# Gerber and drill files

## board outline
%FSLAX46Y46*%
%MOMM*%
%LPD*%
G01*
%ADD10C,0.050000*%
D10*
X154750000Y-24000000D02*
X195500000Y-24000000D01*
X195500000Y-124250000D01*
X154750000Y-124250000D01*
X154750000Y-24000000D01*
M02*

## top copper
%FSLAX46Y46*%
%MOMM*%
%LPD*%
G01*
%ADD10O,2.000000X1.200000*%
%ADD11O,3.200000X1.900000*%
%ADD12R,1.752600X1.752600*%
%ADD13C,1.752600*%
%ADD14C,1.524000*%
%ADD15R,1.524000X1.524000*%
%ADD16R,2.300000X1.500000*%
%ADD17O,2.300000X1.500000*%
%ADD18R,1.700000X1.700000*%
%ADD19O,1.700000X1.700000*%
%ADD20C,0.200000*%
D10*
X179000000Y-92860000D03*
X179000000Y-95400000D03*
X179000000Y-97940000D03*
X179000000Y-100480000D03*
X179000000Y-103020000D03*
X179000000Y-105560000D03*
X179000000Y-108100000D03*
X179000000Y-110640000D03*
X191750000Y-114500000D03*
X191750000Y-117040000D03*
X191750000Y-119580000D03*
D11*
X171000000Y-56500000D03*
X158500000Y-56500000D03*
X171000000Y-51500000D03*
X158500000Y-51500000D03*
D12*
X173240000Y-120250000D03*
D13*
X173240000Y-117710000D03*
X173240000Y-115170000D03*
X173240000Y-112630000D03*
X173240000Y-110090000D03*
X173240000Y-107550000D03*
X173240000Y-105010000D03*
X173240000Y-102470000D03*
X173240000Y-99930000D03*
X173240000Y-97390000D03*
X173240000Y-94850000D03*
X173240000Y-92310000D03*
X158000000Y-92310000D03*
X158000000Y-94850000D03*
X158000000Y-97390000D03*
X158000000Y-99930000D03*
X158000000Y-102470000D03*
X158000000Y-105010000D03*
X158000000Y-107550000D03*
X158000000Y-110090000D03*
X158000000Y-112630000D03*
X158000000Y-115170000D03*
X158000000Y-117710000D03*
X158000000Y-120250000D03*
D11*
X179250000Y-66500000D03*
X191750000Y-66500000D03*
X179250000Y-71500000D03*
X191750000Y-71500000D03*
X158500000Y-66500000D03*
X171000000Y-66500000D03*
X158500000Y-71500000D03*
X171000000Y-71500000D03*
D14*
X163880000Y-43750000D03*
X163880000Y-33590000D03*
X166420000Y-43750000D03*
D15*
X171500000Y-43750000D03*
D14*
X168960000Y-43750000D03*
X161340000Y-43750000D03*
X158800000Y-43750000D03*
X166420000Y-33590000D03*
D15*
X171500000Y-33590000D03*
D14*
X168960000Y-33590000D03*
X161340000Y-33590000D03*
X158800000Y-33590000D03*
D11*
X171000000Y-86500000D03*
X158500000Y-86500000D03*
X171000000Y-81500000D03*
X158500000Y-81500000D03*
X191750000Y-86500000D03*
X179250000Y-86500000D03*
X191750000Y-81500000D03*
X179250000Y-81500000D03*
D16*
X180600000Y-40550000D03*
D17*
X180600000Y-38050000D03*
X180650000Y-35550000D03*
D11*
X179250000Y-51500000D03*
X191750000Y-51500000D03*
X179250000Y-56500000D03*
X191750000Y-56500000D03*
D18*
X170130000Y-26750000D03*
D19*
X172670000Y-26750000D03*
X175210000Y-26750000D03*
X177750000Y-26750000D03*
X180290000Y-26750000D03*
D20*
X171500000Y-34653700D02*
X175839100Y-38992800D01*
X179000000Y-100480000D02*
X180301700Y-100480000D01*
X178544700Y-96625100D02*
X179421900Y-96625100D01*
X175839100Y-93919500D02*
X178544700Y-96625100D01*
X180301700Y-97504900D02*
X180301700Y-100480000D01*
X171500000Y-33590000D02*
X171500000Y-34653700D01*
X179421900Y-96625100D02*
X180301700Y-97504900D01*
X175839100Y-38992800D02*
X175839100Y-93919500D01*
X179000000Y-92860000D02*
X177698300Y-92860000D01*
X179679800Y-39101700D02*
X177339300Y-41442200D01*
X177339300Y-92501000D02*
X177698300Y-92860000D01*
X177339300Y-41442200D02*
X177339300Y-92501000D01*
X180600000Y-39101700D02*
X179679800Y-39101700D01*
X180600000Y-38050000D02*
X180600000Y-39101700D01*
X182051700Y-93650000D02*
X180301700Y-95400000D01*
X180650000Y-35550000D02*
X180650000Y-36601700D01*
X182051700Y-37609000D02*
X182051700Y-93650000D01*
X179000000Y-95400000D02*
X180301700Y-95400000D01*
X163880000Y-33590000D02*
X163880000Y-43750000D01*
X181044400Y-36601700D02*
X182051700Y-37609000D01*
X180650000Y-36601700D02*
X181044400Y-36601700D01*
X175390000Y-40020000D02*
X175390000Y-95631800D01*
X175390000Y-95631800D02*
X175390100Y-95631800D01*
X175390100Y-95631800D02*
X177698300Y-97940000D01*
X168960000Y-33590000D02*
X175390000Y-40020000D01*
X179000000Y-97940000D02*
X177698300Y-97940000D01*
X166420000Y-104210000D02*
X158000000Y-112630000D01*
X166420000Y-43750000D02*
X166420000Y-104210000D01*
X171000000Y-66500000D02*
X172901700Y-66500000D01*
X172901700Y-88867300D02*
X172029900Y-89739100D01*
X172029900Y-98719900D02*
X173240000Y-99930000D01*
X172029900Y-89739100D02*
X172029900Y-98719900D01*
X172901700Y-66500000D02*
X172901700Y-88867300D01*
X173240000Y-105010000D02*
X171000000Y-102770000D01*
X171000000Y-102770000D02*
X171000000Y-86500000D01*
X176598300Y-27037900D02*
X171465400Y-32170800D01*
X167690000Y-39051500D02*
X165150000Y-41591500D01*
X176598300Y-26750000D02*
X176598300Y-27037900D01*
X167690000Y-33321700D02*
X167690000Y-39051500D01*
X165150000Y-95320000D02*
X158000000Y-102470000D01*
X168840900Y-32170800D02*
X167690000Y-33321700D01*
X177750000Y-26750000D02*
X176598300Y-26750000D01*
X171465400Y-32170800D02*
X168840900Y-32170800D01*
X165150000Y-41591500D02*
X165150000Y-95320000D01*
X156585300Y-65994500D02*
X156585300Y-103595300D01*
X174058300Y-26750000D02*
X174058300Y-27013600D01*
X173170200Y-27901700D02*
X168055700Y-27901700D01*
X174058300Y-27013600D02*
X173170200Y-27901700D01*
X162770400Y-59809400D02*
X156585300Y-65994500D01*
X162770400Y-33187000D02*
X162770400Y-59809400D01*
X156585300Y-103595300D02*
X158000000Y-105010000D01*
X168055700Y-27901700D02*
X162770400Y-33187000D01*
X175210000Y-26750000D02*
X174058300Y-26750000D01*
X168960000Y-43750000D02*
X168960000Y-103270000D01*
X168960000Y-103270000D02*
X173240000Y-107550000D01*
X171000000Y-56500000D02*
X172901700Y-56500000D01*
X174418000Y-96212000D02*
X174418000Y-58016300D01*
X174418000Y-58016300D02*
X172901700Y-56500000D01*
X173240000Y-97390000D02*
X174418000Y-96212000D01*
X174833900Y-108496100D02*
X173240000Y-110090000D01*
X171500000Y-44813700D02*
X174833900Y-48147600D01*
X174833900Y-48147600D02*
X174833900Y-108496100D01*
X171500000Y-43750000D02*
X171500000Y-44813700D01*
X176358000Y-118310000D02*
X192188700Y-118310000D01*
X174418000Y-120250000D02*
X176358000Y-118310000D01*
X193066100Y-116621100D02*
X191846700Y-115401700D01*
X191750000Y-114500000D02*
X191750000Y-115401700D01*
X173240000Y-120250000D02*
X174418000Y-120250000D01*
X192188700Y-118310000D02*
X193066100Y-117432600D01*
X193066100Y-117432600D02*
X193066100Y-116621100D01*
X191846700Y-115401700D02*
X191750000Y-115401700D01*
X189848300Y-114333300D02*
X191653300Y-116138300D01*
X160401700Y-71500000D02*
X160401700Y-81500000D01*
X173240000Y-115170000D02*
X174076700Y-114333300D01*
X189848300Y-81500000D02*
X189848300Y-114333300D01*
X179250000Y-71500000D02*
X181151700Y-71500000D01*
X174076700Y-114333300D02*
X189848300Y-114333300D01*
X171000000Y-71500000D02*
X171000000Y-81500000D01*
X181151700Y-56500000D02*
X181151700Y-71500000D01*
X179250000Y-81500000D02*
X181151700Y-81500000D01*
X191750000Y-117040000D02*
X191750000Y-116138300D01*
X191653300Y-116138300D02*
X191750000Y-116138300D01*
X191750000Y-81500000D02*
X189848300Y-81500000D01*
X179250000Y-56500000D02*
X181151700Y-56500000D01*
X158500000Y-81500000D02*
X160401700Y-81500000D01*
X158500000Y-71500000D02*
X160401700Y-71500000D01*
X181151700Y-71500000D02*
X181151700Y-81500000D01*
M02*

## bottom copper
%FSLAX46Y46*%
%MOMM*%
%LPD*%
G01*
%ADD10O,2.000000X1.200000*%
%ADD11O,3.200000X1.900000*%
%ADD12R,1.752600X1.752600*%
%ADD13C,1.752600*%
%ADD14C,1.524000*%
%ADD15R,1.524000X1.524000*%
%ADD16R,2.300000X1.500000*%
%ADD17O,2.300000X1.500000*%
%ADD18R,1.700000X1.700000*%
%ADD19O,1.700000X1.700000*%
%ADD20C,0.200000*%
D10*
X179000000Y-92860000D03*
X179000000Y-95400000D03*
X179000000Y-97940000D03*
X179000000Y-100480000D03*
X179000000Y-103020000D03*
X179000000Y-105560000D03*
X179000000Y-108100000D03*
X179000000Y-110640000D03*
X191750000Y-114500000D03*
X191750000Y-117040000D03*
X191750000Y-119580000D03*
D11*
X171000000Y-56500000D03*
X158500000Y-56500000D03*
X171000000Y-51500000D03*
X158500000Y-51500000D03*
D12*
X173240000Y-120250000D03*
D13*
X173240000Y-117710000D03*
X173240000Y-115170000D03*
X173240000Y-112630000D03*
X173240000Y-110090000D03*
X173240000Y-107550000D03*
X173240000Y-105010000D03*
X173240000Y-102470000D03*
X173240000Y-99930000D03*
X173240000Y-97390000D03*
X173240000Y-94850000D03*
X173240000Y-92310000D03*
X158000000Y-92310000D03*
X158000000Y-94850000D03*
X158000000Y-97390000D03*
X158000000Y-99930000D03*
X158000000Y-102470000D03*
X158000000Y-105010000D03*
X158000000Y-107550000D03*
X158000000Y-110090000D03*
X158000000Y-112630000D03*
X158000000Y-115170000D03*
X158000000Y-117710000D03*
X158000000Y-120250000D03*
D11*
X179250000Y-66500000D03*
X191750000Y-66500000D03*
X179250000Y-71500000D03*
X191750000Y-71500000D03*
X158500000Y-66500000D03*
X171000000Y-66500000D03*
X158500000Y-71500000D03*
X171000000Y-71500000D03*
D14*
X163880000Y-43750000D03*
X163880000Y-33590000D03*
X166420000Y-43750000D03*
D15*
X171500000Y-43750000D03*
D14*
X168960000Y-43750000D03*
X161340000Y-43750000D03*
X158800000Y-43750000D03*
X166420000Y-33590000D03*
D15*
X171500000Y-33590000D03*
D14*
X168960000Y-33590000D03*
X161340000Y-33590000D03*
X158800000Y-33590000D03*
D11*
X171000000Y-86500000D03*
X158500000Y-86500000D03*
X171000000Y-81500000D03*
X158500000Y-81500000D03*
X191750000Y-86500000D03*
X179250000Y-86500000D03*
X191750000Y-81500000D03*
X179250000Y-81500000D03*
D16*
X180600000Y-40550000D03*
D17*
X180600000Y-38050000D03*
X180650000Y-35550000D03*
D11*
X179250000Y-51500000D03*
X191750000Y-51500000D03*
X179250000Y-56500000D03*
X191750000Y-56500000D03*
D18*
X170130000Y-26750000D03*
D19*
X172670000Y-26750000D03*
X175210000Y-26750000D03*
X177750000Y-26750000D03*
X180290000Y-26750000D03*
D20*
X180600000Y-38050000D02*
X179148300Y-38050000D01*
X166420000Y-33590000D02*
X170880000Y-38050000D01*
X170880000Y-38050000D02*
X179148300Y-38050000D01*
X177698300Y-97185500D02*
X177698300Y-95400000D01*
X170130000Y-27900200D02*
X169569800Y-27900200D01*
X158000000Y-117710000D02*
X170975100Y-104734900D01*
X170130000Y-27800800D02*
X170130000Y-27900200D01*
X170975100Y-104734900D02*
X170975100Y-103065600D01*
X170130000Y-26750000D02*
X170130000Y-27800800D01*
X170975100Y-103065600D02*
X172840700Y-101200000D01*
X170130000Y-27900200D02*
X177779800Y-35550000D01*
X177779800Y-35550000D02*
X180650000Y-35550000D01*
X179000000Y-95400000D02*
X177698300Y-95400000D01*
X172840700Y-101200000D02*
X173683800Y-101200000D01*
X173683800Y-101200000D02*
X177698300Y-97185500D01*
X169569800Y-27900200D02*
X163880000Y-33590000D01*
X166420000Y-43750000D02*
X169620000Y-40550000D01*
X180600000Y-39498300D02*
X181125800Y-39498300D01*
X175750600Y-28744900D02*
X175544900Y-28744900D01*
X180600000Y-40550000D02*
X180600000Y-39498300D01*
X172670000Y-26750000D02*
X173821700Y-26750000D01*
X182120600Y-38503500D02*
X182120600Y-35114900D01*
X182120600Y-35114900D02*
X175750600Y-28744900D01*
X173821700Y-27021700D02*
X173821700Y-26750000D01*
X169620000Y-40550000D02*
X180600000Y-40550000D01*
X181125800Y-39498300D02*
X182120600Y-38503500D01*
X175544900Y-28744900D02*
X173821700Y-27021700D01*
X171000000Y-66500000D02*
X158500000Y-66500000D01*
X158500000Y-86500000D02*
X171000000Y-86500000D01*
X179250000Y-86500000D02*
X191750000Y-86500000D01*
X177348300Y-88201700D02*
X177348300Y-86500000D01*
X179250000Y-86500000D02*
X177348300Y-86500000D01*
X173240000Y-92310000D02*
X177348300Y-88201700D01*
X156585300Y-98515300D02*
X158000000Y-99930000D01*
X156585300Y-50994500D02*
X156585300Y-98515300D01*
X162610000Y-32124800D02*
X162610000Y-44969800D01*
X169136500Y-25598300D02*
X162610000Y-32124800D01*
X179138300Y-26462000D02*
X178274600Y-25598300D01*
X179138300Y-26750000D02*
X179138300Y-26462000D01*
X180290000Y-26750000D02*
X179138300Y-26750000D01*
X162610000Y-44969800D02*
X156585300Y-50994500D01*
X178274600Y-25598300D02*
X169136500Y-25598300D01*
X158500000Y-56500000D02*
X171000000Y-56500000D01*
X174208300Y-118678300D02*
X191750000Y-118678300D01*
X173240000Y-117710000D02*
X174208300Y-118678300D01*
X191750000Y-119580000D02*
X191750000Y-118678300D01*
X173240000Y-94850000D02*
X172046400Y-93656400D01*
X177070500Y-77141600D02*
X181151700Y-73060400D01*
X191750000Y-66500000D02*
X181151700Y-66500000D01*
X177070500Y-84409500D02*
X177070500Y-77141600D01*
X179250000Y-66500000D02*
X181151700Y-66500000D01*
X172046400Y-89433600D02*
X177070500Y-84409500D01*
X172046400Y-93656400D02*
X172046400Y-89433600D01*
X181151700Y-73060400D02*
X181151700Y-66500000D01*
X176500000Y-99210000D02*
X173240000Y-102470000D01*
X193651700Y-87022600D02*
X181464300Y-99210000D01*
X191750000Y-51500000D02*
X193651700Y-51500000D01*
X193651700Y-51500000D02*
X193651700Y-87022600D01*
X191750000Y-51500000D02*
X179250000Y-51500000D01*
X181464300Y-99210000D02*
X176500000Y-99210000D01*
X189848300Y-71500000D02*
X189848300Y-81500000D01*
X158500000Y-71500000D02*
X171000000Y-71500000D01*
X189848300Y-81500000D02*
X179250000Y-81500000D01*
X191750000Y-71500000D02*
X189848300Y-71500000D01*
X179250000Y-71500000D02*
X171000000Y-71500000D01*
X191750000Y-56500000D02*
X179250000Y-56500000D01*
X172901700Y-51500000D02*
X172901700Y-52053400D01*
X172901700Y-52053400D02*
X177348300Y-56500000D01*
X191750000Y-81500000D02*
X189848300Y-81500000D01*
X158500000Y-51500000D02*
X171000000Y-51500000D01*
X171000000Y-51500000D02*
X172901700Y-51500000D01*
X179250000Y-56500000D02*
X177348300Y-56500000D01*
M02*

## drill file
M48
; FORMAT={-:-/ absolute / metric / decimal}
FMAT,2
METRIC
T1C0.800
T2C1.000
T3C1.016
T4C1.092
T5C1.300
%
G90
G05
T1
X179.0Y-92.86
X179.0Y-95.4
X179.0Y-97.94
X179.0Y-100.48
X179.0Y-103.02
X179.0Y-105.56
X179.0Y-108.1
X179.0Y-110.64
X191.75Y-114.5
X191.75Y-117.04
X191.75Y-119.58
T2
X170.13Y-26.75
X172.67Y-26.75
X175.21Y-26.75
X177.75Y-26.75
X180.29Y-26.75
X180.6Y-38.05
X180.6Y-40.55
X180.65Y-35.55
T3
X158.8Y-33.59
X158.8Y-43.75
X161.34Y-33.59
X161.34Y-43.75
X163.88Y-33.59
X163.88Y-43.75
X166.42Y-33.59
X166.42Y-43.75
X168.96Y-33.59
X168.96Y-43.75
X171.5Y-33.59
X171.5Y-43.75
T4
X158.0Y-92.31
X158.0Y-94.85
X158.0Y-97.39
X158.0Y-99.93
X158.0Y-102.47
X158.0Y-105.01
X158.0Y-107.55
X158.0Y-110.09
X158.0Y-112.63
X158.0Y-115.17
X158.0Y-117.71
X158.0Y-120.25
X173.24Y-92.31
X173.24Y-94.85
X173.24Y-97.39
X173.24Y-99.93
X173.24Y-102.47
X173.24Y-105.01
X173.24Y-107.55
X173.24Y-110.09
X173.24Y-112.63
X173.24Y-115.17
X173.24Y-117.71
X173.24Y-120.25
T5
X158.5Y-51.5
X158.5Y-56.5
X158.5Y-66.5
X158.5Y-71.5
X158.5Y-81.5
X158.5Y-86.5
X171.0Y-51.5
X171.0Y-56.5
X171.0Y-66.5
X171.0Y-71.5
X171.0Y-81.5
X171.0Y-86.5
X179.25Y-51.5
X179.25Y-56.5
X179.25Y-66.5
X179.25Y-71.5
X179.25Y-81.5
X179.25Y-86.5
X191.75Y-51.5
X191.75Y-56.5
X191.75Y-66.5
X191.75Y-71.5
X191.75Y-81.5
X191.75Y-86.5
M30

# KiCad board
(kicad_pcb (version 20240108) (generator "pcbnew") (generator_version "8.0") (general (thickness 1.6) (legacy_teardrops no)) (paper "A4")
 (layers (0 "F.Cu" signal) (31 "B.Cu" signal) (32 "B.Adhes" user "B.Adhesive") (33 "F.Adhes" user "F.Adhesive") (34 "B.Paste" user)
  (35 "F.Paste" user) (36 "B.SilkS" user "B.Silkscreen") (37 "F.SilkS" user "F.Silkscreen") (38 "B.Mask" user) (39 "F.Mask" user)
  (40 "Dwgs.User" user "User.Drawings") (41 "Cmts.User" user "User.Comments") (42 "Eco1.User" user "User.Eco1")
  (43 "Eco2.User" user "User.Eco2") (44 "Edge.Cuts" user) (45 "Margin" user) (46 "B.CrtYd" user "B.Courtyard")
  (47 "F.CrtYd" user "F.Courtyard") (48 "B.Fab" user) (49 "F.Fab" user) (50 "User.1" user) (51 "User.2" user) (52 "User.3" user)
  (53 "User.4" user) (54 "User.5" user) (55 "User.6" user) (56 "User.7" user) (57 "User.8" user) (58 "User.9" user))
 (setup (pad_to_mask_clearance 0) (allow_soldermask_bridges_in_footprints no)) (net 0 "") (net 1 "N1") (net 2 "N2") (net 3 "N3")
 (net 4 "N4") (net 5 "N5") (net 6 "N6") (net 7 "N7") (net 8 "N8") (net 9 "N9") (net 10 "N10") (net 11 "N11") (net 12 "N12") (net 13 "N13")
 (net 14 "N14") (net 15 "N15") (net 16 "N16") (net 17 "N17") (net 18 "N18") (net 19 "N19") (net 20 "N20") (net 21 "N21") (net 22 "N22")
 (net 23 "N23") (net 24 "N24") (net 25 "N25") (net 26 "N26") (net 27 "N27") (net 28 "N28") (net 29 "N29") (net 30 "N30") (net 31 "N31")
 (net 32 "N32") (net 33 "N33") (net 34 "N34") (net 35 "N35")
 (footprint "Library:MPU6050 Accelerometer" (layer "F.Cu") (at 185.5 104)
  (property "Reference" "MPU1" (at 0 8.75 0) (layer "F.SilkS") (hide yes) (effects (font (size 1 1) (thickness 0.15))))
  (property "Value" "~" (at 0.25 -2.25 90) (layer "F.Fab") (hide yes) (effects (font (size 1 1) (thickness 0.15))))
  (pad "1" thru_hole oval (at -6.5 -11.14 270) (size 1.2 2) (drill 0.8) (layers "*.Cu" "*.Mask") (remove_unused_layers no) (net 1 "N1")
   (thermal_bridge_angle 45))
  (pad "2" thru_hole oval (at -6.5 -8.6 270) (size 1.2 2) (drill 0.8) (layers "*.Cu" "*.Mask") (remove_unused_layers no) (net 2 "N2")
   (thermal_bridge_angle 45))
  (pad "3" thru_hole oval (at -6.5 -6.06 270) (size 1.2 2) (drill 0.8) (layers "*.Cu" "*.Mask") (remove_unused_layers no) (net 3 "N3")
   (thermal_bridge_angle 45))
  (pad "4" thru_hole oval (at -6.5 -3.52 270) (size 1.2 2) (drill 0.8) (layers "*.Cu" "*.Mask") (remove_unused_layers no) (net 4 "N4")
   (thermal_bridge_angle 45))
  (pad "5" thru_hole oval (at -6.5 -0.98 270) (size 1.2 2) (drill 0.8) (layers "*.Cu" "*.Mask") (remove_unused_layers no) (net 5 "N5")
   (thermal_bridge_angle 45))
  (pad "6" thru_hole oval (at -6.5 1.56 270) (size 1.2 2) (drill 0.8) (layers "*.Cu" "*.Mask") (remove_unused_layers no) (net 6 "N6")
   (thermal_bridge_angle 45))
  (pad "7" thru_hole oval (at -6.5 4.1 270) (size 1.2 2) (drill 0.8) (layers "*.Cu" "*.Mask") (remove_unused_layers no) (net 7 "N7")
   (thermal_bridge_angle 45))
  (pad "8" thru_hole oval (at -6.5 6.64 270) (size 1.2 2) (drill 0.8) (layers "*.Cu" "*.Mask") (remove_unused_layers no) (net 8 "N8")
   (thermal_bridge_angle 45)))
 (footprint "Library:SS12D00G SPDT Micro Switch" (layer "F.Cu") (at 191.75 117.04 -90)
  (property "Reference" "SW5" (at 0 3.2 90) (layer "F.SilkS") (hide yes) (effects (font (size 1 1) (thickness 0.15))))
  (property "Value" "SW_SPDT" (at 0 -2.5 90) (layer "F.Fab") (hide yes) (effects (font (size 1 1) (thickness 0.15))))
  (pad "1" thru_hole oval (at -2.54 0 270) (size 1.2 2) (drill 0.8) (layers "*.Cu" "*.Mask") (remove_unused_layers no) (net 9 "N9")
   (thermal_bridge_angle 45))
  (pad "2" thru_hole oval (at 0 0 270) (size 1.2 2) (drill 0.8) (layers "*.Cu" "*.Mask") (remove_unused_layers no) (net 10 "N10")
   (thermal_bridge_angle 45))
  (pad "3" thru_hole oval (at 2.54 0 270) (size 1.2 2) (drill 0.8) (layers "*.Cu" "*.Mask") (remove_unused_layers no) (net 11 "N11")
   (thermal_bridge_angle 45)))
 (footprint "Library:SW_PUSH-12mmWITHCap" (layer "F.Cu") (at 171 56.5 180)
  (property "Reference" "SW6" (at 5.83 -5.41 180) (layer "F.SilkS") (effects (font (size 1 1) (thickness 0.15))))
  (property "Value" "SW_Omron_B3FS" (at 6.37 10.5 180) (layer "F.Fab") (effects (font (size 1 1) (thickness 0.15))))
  (pad "1" thru_hole oval (at 0 0 180) (size 3.2 1.9) (drill 1.3) (layers "*.Cu" "*.Mask") (remove_unused_layers no) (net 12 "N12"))
  (pad "1" thru_hole oval (at 12.5 0 180) (size 3.2 1.9) (drill 1.3) (layers "*.Cu" "*.Mask") (remove_unused_layers no) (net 12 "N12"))
  (pad "2" thru_hole oval (at 0 5 180) (size 3.2 1.9) (drill 1.3) (layers "*.Cu" "*.Mask") (remove_unused_layers no) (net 10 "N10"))
  (pad "2" thru_hole oval (at 12.5 5 180) (size 3.2 1.9) (drill 1.3) (layers "*.Cu" "*.Mask") (remove_unused_layers no) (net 10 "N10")))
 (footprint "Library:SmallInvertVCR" (layer "F.Cu") (at 182.25 117.5)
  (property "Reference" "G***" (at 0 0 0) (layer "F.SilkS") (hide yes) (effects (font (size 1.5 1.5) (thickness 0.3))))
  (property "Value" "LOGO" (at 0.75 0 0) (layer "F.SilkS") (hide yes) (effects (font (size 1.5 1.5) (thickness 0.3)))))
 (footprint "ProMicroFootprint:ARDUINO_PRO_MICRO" (layer "F.Cu") (at 165.62 106.28 90)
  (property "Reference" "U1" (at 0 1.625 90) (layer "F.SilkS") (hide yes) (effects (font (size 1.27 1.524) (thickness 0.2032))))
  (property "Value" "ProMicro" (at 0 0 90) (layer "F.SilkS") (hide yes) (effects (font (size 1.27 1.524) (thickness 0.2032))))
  (pad "1" thru_hole rect (at -13.97 7.62 90) (size 1.7526 1.7526) (drill 1.0922) (layers "*.Cu" "*.SilkS" "*.Mask")
   (remove_unused_layers no) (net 9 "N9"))
  (pad "2" thru_hole circle (at -11.43 7.62 90) (size 1.7526 1.7526) (drill 1.0922) (layers "*.Cu" "*.SilkS" "*.Mask")
   (remove_unused_layers no) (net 11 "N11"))
  (pad "3" thru_hole circle (at -8.89 7.62 90) (size 1.7526 1.7526) (drill 1.0922) (layers "*.Cu" "*.SilkS" "*.Mask")
   (remove_unused_layers no) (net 10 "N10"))
  (pad "4" thru_hole circle (at -6.35 7.62 90) (size 1.7526 1.7526) (drill 1.0922) (layers "*.Cu" "*.SilkS" "*.Mask")
   (remove_unused_layers no) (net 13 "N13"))
  (pad "5" thru_hole circle (at -3.81 7.62 90) (size 1.7526 1.7526) (drill 1.0922) (layers "*.Cu" "*.SilkS" "*.Mask")
   (remove_unused_layers no) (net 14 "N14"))
  (pad "6" thru_hole circle (at -1.27 7.62 90) (size 1.7526 1.7526) (drill 1.0922) (layers "*.Cu" "*.SilkS" "*.Mask")
   (remove_unused_layers no) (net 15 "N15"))
  (pad "7" thru_hole circle (at 1.27 7.62 90) (size 1.7526 1.7526) (drill 1.0922) (layers "*.Cu" "*.SilkS" "*.Mask")
   (remove_unused_layers no) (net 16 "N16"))
  (pad "8" thru_hole circle (at 3.81 7.62 90) (size 1.7526 1.7526) (drill 1.0922) (layers "*.Cu" "*.SilkS" "*.Mask")
   (remove_unused_layers no) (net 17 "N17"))
  (pad "9" thru_hole circle (at 6.35 7.62 90) (size 1.7526 1.7526) (drill 1.0922) (layers "*.Cu" "*.SilkS" "*.Mask")
   (remove_unused_layers no) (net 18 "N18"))
  (pad "10" thru_hole circle (at 8.89 7.62 90) (size 1.7526 1.7526) (drill 1.0922) (layers "*.Cu" "*.SilkS" "*.Mask")
   (remove_unused_layers no) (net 12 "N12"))
  (pad "11" thru_hole circle (at 11.43 7.62 90) (size 1.7526 1.7526) (drill 1.0922) (layers "*.Cu" "*.SilkS" "*.Mask")
   (remove_unused_layers no) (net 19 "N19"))
  (pad "12" thru_hole circle (at 13.97 7.62 90) (size 1.7526 1.7526) (drill 1.0922) (layers "*.Cu" "*.SilkS" "*.Mask")
   (remove_unused_layers no) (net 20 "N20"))
  (pad "13" thru_hole circle (at 13.97 -7.62 90) (size 1.7526 1.7526) (drill 1.0922) (layers "*.Cu" "*.SilkS" "*.Mask")
   (remove_unused_layers no) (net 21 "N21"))
  (pad "14" thru_hole circle (at 11.43 -7.62 90) (size 1.7526 1.7526) (drill 1.0922) (layers "*.Cu" "*.SilkS" "*.Mask")
   (remove_unused_layers no) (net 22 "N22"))
  (pad "15" thru_hole circle (at 8.89 -7.62 90) (size 1.7526 1.7526) (drill 1.0922) (layers "*.Cu" "*.SilkS" "*.Mask")
   (remove_unused_layers no) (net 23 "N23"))
  (pad "16" thru_hole circle (at 6.35 -7.62 90) (size 1.7526 1.7526) (drill 1.0922) (layers "*.Cu" "*.SilkS" "*.Mask")
   (remove_unused_layers no) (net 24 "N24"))
  (pad "17" thru_hole circle (at 3.81 -7.62 90) (size 1.7526 1.7526) (drill 1.0922) (layers "*.Cu" "*.SilkS" "*.Mask")
   (remove_unused_layers no) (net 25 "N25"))
  (pad "18" thru_hole circle (at 1.27 -7.62 90) (size 1.7526 1.7526) (drill 1.0922) (layers "*.Cu" "*.SilkS" "*.Mask")
   (remove_unused_layers no) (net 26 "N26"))
  (pad "19" thru_hole circle (at -1.27 -7.62 90) (size 1.7526 1.7526) (drill 1.0922) (layers "*.Cu" "*.SilkS" "*.Mask")
   (remove_unused_layers no) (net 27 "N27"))
  (pad "20" thru_hole circle (at -3.81 -7.62 90) (size 1.7526 1.7526) (drill 1.0922) (layers "*.Cu" "*.SilkS" "*.Mask")
   (remove_unused_layers no) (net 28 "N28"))
  (pad "21" thru_hole circle (at -6.35 -7.62 90) (size 1.7526 1.7526) (drill 1.0922) (layers "*.Cu" "*.SilkS" "*.Mask")
   (remove_unused_layers no) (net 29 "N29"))
  (pad "22" thru_hole circle (at -8.89 -7.62 90) (size 1.7526 1.7526) (drill 1.0922) (layers "*.Cu" "*.SilkS" "*.Mask")
   (remove_unused_layers no) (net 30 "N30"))
  (pad "23" thru_hole circle (at -11.43 -7.62 90) (size 1.7526 1.7526) (drill 1.0922) (layers "*.Cu" "*.SilkS" "*.Mask")
   (remove_unused_layers no) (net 2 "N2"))
  (pad "24" thru_hole circle (at -13.97 -7.62 90) (size 1.7526 1.7526) (drill 1.0922) (layers "*.Cu" "*.SilkS" "*.Mask")
   (remove_unused_layers no) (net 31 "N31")))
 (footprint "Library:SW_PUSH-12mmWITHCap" (layer "F.Cu") (at 179.25 66.5)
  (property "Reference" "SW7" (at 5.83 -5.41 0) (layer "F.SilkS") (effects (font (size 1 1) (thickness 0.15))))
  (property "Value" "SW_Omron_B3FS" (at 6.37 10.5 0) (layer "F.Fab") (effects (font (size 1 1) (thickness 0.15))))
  (pad "1" thru_hole oval (at 0 0) (size 3.2 1.9) (drill 1.3) (layers "*.Cu" "*.Mask") (remove_unused_layers no) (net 19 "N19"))
  (pad "1" thru_hole oval (at 12.5 0) (size 3.2 1.9) (drill 1.3) (layers "*.Cu" "*.Mask") (remove_unused_layers no) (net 19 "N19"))
  (pad "2" thru_hole oval (at 0 5) (size 3.2 1.9) (drill 1.3) (layers "*.Cu" "*.Mask") (remove_unused_layers no) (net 10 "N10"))
  (pad "2" thru_hole oval (at 12.5 5) (size 3.2 1.9) (drill 1.3) (layers "*.Cu" "*.Mask") (remove_unused_layers no) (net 10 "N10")))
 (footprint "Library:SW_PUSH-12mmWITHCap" (layer "F.Cu") (at 158.5 66.5)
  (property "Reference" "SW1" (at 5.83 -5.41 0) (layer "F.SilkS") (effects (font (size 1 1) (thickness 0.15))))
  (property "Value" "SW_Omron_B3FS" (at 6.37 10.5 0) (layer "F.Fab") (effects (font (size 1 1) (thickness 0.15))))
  (pad "1" thru_hole oval (at 0 0) (size 3.2 1.9) (drill 1.3) (layers "*.Cu" "*.Mask") (remove_unused_layers no) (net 18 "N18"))
  (pad "1" thru_hole oval (at 12.5 0) (size 3.2 1.9) (drill 1.3) (layers "*.Cu" "*.Mask") (remove_unused_layers no) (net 18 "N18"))
  (pad "2" thru_hole oval (at 0 5) (size 3.2 1.9) (drill 1.3) (layers "*.Cu" "*.Mask") (remove_unused_layers no) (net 10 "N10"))
  (pad "2" thru_hole oval (at 12.5 5) (size 3.2 1.9) (drill 1.3) (layers "*.Cu" "*.Mask") (remove_unused_layers no) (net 10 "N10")))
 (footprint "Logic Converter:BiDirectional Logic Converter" (layer "F.Cu") (at 165.15 38.67 -90)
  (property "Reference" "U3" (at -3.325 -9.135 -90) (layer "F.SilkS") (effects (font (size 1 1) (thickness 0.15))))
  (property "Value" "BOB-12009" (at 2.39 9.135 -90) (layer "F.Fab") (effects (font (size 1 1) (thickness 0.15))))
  (pad "GND_1" thru_hole circle (at 5.08 1.27 270) (size 1.524 1.524) (drill 1.016) (layers "*.Cu" "*.Mask") (remove_unused_layers no)
   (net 2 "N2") (solder_mask_margin 0.102))
  (pad "GND_2" thru_hole circle (at -5.08 1.27 270) (size 1.524 1.524) (drill 1.016) (layers "*.Cu" "*.Mask") (remove_unused_layers no)
   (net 2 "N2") (solder_mask_margin 0.102))
  (pad "HV" thru_hole circle (at 5.08 -1.27 270) (size 1.524 1.524) (drill 1.016) (layers "*.Cu" "*.Mask") (remove_unused_layers no)
   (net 29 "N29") (solder_mask_margin 0.102))
  (pad "HV1" thru_hole rect (at 5.08 -6.35 270) (size 1.524 1.524) (drill 1.016) (layers "*.Cu" "*.Mask") (remove_unused_layers no)
   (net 14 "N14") (solder_mask_margin 0.102))
  (pad "HV2" thru_hole circle (at 5.08 -3.81 270) (size 1.524 1.524) (drill 1.016) (layers "*.Cu" "*.Mask") (remove_unused_layers no)
   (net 15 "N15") (solder_mask_margin 0.102))
  (pad "HV3" thru_hole circle (at 5.08 3.81 270) (size 1.524 1.524) (drill 1.016) (layers "*.Cu" "*.Mask") (remove_unused_layers no)
   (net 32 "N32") (solder_mask_margin 0.102))
  (pad "HV4" thru_hole circle (at 5.08 6.35 270) (size 1.524 1.524) (drill 1.016) (layers "*.Cu" "*.Mask") (remove_unused_layers no)
   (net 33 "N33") (solder_mask_margin 0.102))
  (pad "LV" thru_hole circle (at -5.08 -1.27 270) (size 1.524 1.524) (drill 1.016) (layers "*.Cu" "*.Mask") (remove_unused_layers no)
   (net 1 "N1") (solder_mask_margin 0.102))
  (pad "LV1" thru_hole rect (at -5.08 -6.35 270) (size 1.524 1.524) (drill 1.016) (layers "*.Cu" "*.Mask") (remove_unused_layers no)
   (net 4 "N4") (solder_mask_margin 0.102))
  (pad "LV2" thru_hole circle (at -5.08 -3.81 270) (size 1.524 1.524) (drill 1.016) (layers "*.Cu" "*.Mask") (remove_unused_layers no)
   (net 3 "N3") (solder_mask_margin 0.102))
  (pad "LV3" thru_hole circle (at -5.08 3.81 270) (size 1.524 1.524) (drill 1.016) (layers "*.Cu" "*.Mask") (remove_unused_layers no)
   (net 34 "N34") (solder_mask_margin 0.102))
  (pad "LV4" thru_hole circle (at -5.08 6.35 270) (size 1.524 1.524) (drill 1.016) (layers "*.Cu" "*.Mask") (remove_unused_layers no)
   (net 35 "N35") (solder_mask_margin 0.102)))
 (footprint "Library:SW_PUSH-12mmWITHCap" (layer "F.Cu") (at 171 86.5 180)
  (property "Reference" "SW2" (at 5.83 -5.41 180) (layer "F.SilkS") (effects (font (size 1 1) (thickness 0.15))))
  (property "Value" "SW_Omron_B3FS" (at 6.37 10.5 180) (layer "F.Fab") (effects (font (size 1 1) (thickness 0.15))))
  (pad "1" thru_hole oval (at 0 0 180) (size 3.2 1.9) (drill 1.3) (layers "*.Cu" "*.Mask") (remove_unused_layers no) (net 16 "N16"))
  (pad "1" thru_hole oval (at 12.5 0 180) (size 3.2 1.9) (drill 1.3) (layers "*.Cu" "*.Mask") (remove_unused_layers no) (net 16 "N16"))
  (pad "2" thru_hole oval (at 0 5 180) (size 3.2 1.9) (drill 1.3) (layers "*.Cu" "*.Mask") (remove_unused_layers no) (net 10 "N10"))
  (pad "2" thru_hole oval (at 12.5 5 180) (size 3.2 1.9) (drill 1.3) (layers "*.Cu" "*.Mask") (remove_unused_layers no) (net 10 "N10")))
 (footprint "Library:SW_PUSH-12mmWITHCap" (layer "F.Cu") (at 191.75 86.5 180)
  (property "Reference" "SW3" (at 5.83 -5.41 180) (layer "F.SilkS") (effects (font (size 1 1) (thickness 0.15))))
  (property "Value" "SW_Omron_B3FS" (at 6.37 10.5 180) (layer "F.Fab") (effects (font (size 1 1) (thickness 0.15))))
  (pad "1" thru_hole oval (at 0 0 180) (size 3.2 1.9) (drill 1.3) (layers "*.Cu" "*.Mask") (remove_unused_layers no) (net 20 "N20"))
  (pad "1" thru_hole oval (at 12.5 0 180) (size 3.2 1.9) (drill 1.3) (layers "*.Cu" "*.Mask") (remove_unused_layers no) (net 20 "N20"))
  (pad "2" thru_hole oval (at 0 5 180) (size 3.2 1.9) (drill 1.3) (layers "*.Cu" "*.Mask") (remove_unused_layers no) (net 10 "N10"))
  (pad "2" thru_hole oval (at 12.5 5 180) (size 3.2 1.9) (drill 1.3) (layers "*.Cu" "*.Mask") (remove_unused_layers no) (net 10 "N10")))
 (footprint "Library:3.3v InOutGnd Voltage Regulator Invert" (layer "F.Cu") (at 179.1 38 -90)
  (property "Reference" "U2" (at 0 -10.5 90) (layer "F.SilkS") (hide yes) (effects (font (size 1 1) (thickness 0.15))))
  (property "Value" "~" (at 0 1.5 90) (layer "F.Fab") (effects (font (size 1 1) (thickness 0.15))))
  (pad "1" thru_hole rect (at 2.55 -1.5 270) (size 1.5 2.3) (drill 1) (layers "*.Cu" "*.Mask") (remove_unused_layers no) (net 29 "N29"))
  (pad "2" thru_hole oval (at 0.05 -1.5 270) (size 1.5 2.3) (drill 1) (layers "*.Cu" "*.Mask") (remove_unused_layers no) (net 1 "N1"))
  (pad "3" thru_hole oval (at -2.45 -1.55 270) (size 1.5 2.3) (drill 1) (layers "*.Cu" "*.Mask") (remove_unused_layers no) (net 2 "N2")))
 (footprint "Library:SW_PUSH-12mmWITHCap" (layer "F.Cu") (at 179.25 51.5)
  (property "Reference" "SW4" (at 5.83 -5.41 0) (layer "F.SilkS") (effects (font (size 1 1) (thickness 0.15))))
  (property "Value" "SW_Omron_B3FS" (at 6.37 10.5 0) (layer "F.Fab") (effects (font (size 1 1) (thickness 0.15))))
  (pad "1" thru_hole oval (at 0 0) (size 3.2 1.9) (drill 1.3) (layers "*.Cu" "*.Mask") (remove_unused_layers no) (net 17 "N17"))
  (pad "1" thru_hole oval (at 12.5 0) (size 3.2 1.9) (drill 1.3) (layers "*.Cu" "*.Mask") (remove_unused_layers no) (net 17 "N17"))
  (pad "2" thru_hole oval (at 0 5) (size 3.2 1.9) (drill 1.3) (layers "*.Cu" "*.Mask") (remove_unused_layers no) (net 10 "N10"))
  (pad "2" thru_hole oval (at 12.5 5) (size 3.2 1.9) (drill 1.3) (layers "*.Cu" "*.Mask") (remove_unused_layers no) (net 10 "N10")))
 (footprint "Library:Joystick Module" (layer "B.Cu") (at 170.13 26.75 -90)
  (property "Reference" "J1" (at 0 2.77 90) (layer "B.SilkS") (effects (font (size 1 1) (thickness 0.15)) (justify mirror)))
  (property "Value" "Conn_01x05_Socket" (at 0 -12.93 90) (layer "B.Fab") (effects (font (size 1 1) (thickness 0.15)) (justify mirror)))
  (pad "1" thru_hole rect (at 0 0 270) (size 1.7 1.7) (drill 1) (layers "*.Cu" "*.Mask") (remove_unused_layers no) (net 2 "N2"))
  (pad "2" thru_hole oval (at 0 -2.54 270) (size 1.7 1.7) (drill 1) (layers "*.Cu" "*.Mask") (remove_unused_layers no) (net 29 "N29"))
  (pad "3" thru_hole oval (at 0 -5.08 270) (size 1.7 1.7) (drill 1) (layers "*.Cu" "*.Mask") (remove_unused_layers no) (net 26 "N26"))
  (pad "4" thru_hole oval (at 0 -7.62 270) (size 1.7 1.7) (drill 1) (layers "*.Cu" "*.Mask") (remove_unused_layers no) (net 25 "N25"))
  (pad "5" thru_hole oval (at 0 -10.16 270) (size 1.7 1.7) (drill 1) (layers "*.Cu" "*.Mask") (remove_unused_layers no) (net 24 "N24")))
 (gr_rect (start 154.75 24) (end 195.5 124.25) (stroke (width 0.05) (type default)) (fill none) (layer "Edge.Cuts"))
 (segment (start 171.5 34.6537) (end 175.8391 38.9928) (width 0.2) (layer "F.Cu") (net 4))
 (segment (start 179 100.48) (end 180.3017 100.48) (width 0.2) (layer "F.Cu") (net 4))
 (segment (start 178.5447 96.6251) (end 179.4219 96.6251) (width 0.2) (layer "F.Cu") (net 4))
 (segment (start 175.8391 93.9195) (end 178.5447 96.6251) (width 0.2) (layer "F.Cu") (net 4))
 (segment (start 180.3017 97.5049) (end 180.3017 100.48) (width 0.2) (layer "F.Cu") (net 4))
 (segment (start 171.5 33.59) (end 171.5 34.6537) (width 0.2) (layer "F.Cu") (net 4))
 (segment (start 179.4219 96.6251) (end 180.3017 97.5049) (width 0.2) (layer "F.Cu") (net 4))
 (segment (start 175.8391 38.9928) (end 175.8391 93.9195) (width 0.2) (layer "F.Cu") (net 4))
 (segment (start 179 92.86) (end 177.6983 92.86) (width 0.2) (layer "F.Cu") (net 1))
 (segment (start 179.6798 39.1017) (end 177.3393 41.4422) (width 0.2) (layer "F.Cu") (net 1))
 (segment (start 177.3393 92.501) (end 177.6983 92.86) (width 0.2) (layer "F.Cu") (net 1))
 (segment (start 177.3393 41.4422) (end 177.3393 92.501) (width 0.2) (layer "F.Cu") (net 1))
 (segment (start 180.6 39.1017) (end 179.6798 39.1017) (width 0.2) (layer "F.Cu") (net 1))
 (segment (start 180.6 38.05) (end 180.6 39.1017) (width 0.2) (layer "F.Cu") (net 1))
 (segment (start 180.6 38.05) (end 179.1483 38.05) (width 0.2) (layer "B.Cu") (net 1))
 (segment (start 166.42 33.59) (end 170.88 38.05) (width 0.2) (layer "B.Cu") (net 1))
 (segment (start 170.88 38.05) (end 179.1483 38.05) (width 0.2) (layer "B.Cu") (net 1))
 (segment (start 182.0517 93.65) (end 180.3017 95.4) (width 0.2) (layer "F.Cu") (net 2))
 (segment (start 180.65 35.55) (end 180.65 36.6017) (width 0.2) (layer "F.Cu") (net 2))
 (segment (start 182.0517 37.609) (end 182.0517 93.65) (width 0.2) (layer "F.Cu") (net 2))
 (segment (start 179 95.4) (end 180.3017 95.4) (width 0.2) (layer "F.Cu") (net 2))
 (segment (start 163.88 33.59) (end 163.88 43.75) (width 0.2) (layer "F.Cu") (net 2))
 (segment (start 181.0444 36.6017) (end 182.0517 37.609) (width 0.2) (layer "F.Cu") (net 2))
 (segment (start 180.65 36.6017) (end 181.0444 36.6017) (width 0.2) (layer "F.Cu") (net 2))
 (segment (start 177.6983 97.1855) (end 177.6983 95.4) (width 0.2) (layer "B.Cu") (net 2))
 (segment (start 170.13 27.9002) (end 169.5698 27.9002) (width 0.2) (layer "B.Cu") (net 2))
 (segment (start 158 117.71) (end 170.9751 104.7349) (width 0.2) (layer "B.Cu") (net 2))
 (segment (start 170.13 27.8008) (end 170.13 27.9002) (width 0.2) (layer "B.Cu") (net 2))
 (segment (start 170.9751 104.7349) (end 170.9751 103.0656) (width 0.2) (layer "B.Cu") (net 2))
 (segment (start 170.13 26.75) (end 170.13 27.8008) (width 0.2) (layer "B.Cu") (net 2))
 (segment (start 170.9751 103.0656) (end 172.8407 101.2) (width 0.2) (layer "B.Cu") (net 2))
 (segment (start 170.13 27.9002) (end 177.7798 35.55) (width 0.2) (layer "B.Cu") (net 2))
 (segment (start 177.7798 35.55) (end 180.65 35.55) (width 0.2) (layer "B.Cu") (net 2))
 (segment (start 179 95.4) (end 177.6983 95.4) (width 0.2) (layer "B.Cu") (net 2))
 (segment (start 172.8407 101.2) (end 173.6838 101.2) (width 0.2) (layer "B.Cu") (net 2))
 (segment (start 173.6838 101.2) (end 177.6983 97.1855) (width 0.2) (layer "B.Cu") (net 2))
 (segment (start 169.5698 27.9002) (end 163.88 33.59) (width 0.2) (layer "B.Cu") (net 2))
 (segment (start 175.39 40.02) (end 175.39 95.6318) (width 0.2) (layer "F.Cu") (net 3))
 (segment (start 175.39 95.6318) (end 175.3901 95.6318) (width 0.2) (layer "F.Cu") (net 3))
 (segment (start 175.3901 95.6318) (end 177.6983 97.94) (width 0.2) (layer "F.Cu") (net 3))
 (segment (start 168.96 33.59) (end 175.39 40.02) (width 0.2) (layer "F.Cu") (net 3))
 (segment (start 179 97.94) (end 177.6983 97.94) (width 0.2) (layer "F.Cu") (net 3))
 (segment (start 166.42 104.21) (end 158 112.63) (width 0.2) (layer "F.Cu") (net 29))
 (segment (start 166.42 43.75) (end 166.42 104.21) (width 0.2) (layer "F.Cu") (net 29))
 (segment (start 166.42 43.75) (end 169.62 40.55) (width 0.2) (layer "B.Cu") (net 29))
 (segment (start 180.6 39.4983) (end 181.1258 39.4983) (width 0.2) (layer "B.Cu") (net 29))
 (segment (start 175.7506 28.7449) (end 175.5449 28.7449) (width 0.2) (layer "B.Cu") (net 29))
 (segment (start 180.6 40.55) (end 180.6 39.4983) (width 0.2) (layer "B.Cu") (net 29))
 (segment (start 172.67 26.75) (end 173.8217 26.75) (width 0.2) (layer "B.Cu") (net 29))
 (segment (start 182.1206 38.5035) (end 182.1206 35.1149) (width 0.2) (layer "B.Cu") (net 29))
 (segment (start 182.1206 35.1149) (end 175.7506 28.7449) (width 0.2) (layer "B.Cu") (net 29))
 (segment (start 173.8217 27.0217) (end 173.8217 26.75) (width 0.2) (layer "B.Cu") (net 29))
 (segment (start 169.62 40.55) (end 180.6 40.55) (width 0.2) (layer "B.Cu") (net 29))
 (segment (start 181.1258 39.4983) (end 182.1206 38.5035) (width 0.2) (layer "B.Cu") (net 29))
 (segment (start 175.5449 28.7449) (end 173.8217 27.0217) (width 0.2) (layer "B.Cu") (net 29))
 (segment (start 171 66.5) (end 172.9017 66.5) (width 0.2) (layer "F.Cu") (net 18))
 (segment (start 172.9017 88.8673) (end 172.0299 89.7391) (width 0.2) (layer "F.Cu") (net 18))
 (segment (start 172.0299 98.7199) (end 173.24 99.93) (width 0.2) (layer "F.Cu") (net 18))
 (segment (start 172.0299 89.7391) (end 172.0299 98.7199) (width 0.2) (layer "F.Cu") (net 18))
 (segment (start 172.9017 66.5) (end 172.9017 88.8673) (width 0.2) (layer "F.Cu") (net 18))
 (segment (start 171 66.5) (end 158.5 66.5) (width 0.2) (layer "B.Cu") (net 18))
 (segment (start 173.24 105.01) (end 171 102.77) (width 0.2) (layer "F.Cu") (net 16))
 (segment (start 171 102.77) (end 171 86.5) (width 0.2) (layer "F.Cu") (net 16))
 (segment (start 158.5 86.5) (end 171 86.5) (width 0.2) (layer "B.Cu") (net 16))
 (segment (start 179.25 86.5) (end 191.75 86.5) (width 0.2) (layer "B.Cu") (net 20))
 (segment (start 177.3483 88.2017) (end 177.3483 86.5) (width 0.2) (layer "B.Cu") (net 20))
 (segment (start 179.25 86.5) (end 177.3483 86.5) (width 0.2) (layer "B.Cu") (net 20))
 (segment (start 173.24 92.31) (end 177.3483 88.2017) (width 0.2) (layer "B.Cu") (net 20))
 (segment (start 176.5983 27.0379) (end 171.4654 32.1708) (width 0.2) (layer "F.Cu") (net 25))
 (segment (start 167.69 39.0515) (end 165.15 41.5915) (width 0.2) (layer "F.Cu") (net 25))
 (segment (start 176.5983 26.75) (end 176.5983 27.0379) (width 0.2) (layer "F.Cu") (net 25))
 (segment (start 167.69 33.3217) (end 167.69 39.0515) (width 0.2) (layer "F.Cu") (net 25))
 (segment (start 165.15 95.32) (end 158 102.47) (width 0.2) (layer "F.Cu") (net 25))
 (segment (start 168.8409 32.1708) (end 167.69 33.3217) (width 0.2) (layer "F.Cu") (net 25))
 (segment (start 177.75 26.75) (end 176.5983 26.75) (width 0.2) (layer "F.Cu") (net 25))
 (segment (start 171.4654 32.1708) (end 168.8409 32.1708) (width 0.2) (layer "F.Cu") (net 25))
 (segment (start 165.15 41.5915) (end 165.15 95.32) (width 0.2) (layer "F.Cu") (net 25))
 (segment (start 156.5853 98.5153) (end 158 99.93) (width 0.2) (layer "B.Cu") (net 24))
 (segment (start 156.5853 50.9945) (end 156.5853 98.5153) (width 0.2) (layer "B.Cu") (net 24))
 (segment (start 162.61 32.1248) (end 162.61 44.9698) (width 0.2) (layer "B.Cu") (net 24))
 (segment (start 169.1365 25.5983) (end 162.61 32.1248) (width 0.2) (layer "B.Cu") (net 24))
 (segment (start 179.1383 26.462) (end 178.2746 25.5983) (width 0.2) (layer "B.Cu") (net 24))
 (segment (start 179.1383 26.75) (end 179.1383 26.462) (width 0.2) (layer "B.Cu") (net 24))
 (segment (start 180.29 26.75) (end 179.1383 26.75) (width 0.2) (layer "B.Cu") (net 24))
 (segment (start 162.61 44.9698) (end 156.5853 50.9945) (width 0.2) (layer "B.Cu") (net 24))
 (segment (start 178.2746 25.5983) (end 169.1365 25.5983) (width 0.2) (layer "B.Cu") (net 24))
 (segment (start 156.5853 65.9945) (end 156.5853 103.5953) (width 0.2) (layer "F.Cu") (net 26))
 (segment (start 174.0583 26.75) (end 174.0583 27.0136) (width 0.2) (layer "F.Cu") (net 26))
 (segment (start 173.1702 27.9017) (end 168.0557 27.9017) (width 0.2) (layer "F.Cu") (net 26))
 (segment (start 174.0583 27.0136) (end 173.1702 27.9017) (width 0.2) (layer "F.Cu") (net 26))
 (segment (start 162.7704 59.8094) (end 156.5853 65.9945) (width 0.2) (layer "F.Cu") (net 26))
 (segment (start 162.7704 33.187) (end 162.7704 59.8094) (width 0.2) (layer "F.Cu") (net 26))
 (segment (start 156.5853 103.5953) (end 158 105.01) (width 0.2) (layer "F.Cu") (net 26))
 (segment (start 168.0557 27.9017) (end 162.7704 33.187) (width 0.2) (layer "F.Cu") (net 26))
 (segment (start 175.21 26.75) (end 174.0583 26.75) (width 0.2) (layer "F.Cu") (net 26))
 (segment (start 168.96 43.75) (end 168.96 103.27) (width 0.2) (layer "F.Cu") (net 15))
 (segment (start 168.96 103.27) (end 173.24 107.55) (width 0.2) (layer "F.Cu") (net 15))
 (segment (start 171 56.5) (end 172.9017 56.5) (width 0.2) (layer "F.Cu") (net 12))
 (segment (start 174.418 96.212) (end 174.418 58.0163) (width 0.2) (layer "F.Cu") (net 12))
 (segment (start 174.418 58.0163) (end 172.9017 56.5) (width 0.2) (layer "F.Cu") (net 12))
 (segment (start 173.24 97.39) (end 174.418 96.212) (width 0.2) (layer "F.Cu") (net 12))
 (segment (start 158.5 56.5) (end 171 56.5) (width 0.2) (layer "B.Cu") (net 12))
 (segment (start 174.2083 118.6783) (end 191.75 118.6783) (width 0.2) (layer "B.Cu") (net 11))
 (segment (start 173.24 117.71) (end 174.2083 118.6783) (width 0.2) (layer "B.Cu") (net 11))
 (segment (start 191.75 119.58) (end 191.75 118.6783) (width 0.2) (layer "B.Cu") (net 11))
 (segment (start 174.8339 108.4961) (end 173.24 110.09) (width 0.2) (layer "F.Cu") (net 14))
 (segment (start 171.5 44.8137) (end 174.8339 48.1476) (width 0.2) (layer "F.Cu") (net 14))
 (segment (start 174.8339 48.1476) (end 174.8339 108.4961) (width 0.2) (layer "F.Cu") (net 14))
 (segment (start 171.5 43.75) (end 171.5 44.8137) (width 0.2) (layer "F.Cu") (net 14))
 (segment (start 176.358 118.31) (end 192.1887 118.31) (width 0.2) (layer "F.Cu") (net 9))
 (segment (start 174.418 120.25) (end 176.358 118.31) (width 0.2) (layer "F.Cu") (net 9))
 (segment (start 193.0661 116.6211) (end 191.8467 115.4017) (width 0.2) (layer "F.Cu") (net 9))
 (segment (start 191.75 114.5) (end 191.75 115.4017) (width 0.2) (layer "F.Cu") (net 9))
 (segment (start 173.24 120.25) (end 174.418 120.25) (width 0.2) (layer "F.Cu") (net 9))
 (segment (start 192.1887 118.31) (end 193.0661 117.4326) (width 0.2) (layer "F.Cu") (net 9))
 (segment (start 193.0661 117.4326) (end 193.0661 116.6211) (width 0.2) (layer "F.Cu") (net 9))
 (segment (start 191.8467 115.4017) (end 191.75 115.4017) (width 0.2) (layer "F.Cu") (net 9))
 (segment (start 173.24 94.85) (end 172.0464 93.6564) (width 0.2) (layer "B.Cu") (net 19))
 (segment (start 177.0705 77.1416) (end 181.1517 73.0604) (width 0.2) (layer "B.Cu") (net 19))
 (segment (start 191.75 66.5) (end 181.1517 66.5) (width 0.2) (layer "B.Cu") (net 19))
 (segment (start 177.0705 84.4095) (end 177.0705 77.1416) (width 0.2) (layer "B.Cu") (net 19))
 (segment (start 179.25 66.5) (end 181.1517 66.5) (width 0.2) (layer "B.Cu") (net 19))
 (segment (start 172.0464 89.4336) (end 177.0705 84.4095) (width 0.2) (layer "B.Cu") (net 19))
 (segment (start 172.0464 93.6564) (end 172.0464 89.4336) (width 0.2) (layer "B.Cu") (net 19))
 (segment (start 181.1517 73.0604) (end 181.1517 66.5) (width 0.2) (layer "B.Cu") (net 19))
 (segment (start 176.5 99.21) (end 173.24 102.47) (width 0.2) (layer "B.Cu") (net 17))
 (segment (start 193.6517 87.0226) (end 181.4643 99.21) (width 0.2) (layer "B.Cu") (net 17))
 (segment (start 191.75 51.5) (end 193.6517 51.5) (width 0.2) (layer "B.Cu") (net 17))
 (segment (start 193.6517 51.5) (end 193.6517 87.0226) (width 0.2) (layer "B.Cu") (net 17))
 (segment (start 191.75 51.5) (end 179.25 51.5) (width 0.2) (layer "B.Cu") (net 17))
 (segment (start 181.4643 99.21) (end 176.5 99.21) (width 0.2) (layer "B.Cu") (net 17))
 (segment (start 189.8483 114.3333) (end 191.6533 116.1383) (width 0.2) (layer "F.Cu") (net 10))
 (segment (start 160.4017 71.5) (end 160.4017 81.5) (width 0.2) (layer "F.Cu") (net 10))
 (segment (start 173.24 115.17) (end 174.0767 114.3333) (width 0.2) (layer "F.Cu") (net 10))
 (segment (start 189.8483 81.5) (end 189.8483 114.3333) (width 0.2) (layer "F.Cu") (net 10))
 (segment (start 179.25 71.5) (end 181.1517 71.5) (width 0.2) (layer "F.Cu") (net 10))
 (segment (start 174.0767 114.3333) (end 189.8483 114.3333) (width 0.2) (layer "F.Cu") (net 10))
 (segment (start 171 71.5) (end 171 81.5) (width 0.2) (layer "F.Cu") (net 10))
 (segment (start 181.1517 56.5) (end 181.1517 71.5) (width 0.2) (layer "F.Cu") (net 10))
 (segment (start 179.25 81.5) (end 181.1517 81.5) (width 0.2) (layer "F.Cu") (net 10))
 (segment (start 191.75 117.04) (end 191.75 116.1383) (width 0.2) (layer "F.Cu") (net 10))
 (segment (start 191.6533 116.1383) (end 191.75 116.1383) (width 0.2) (layer "F.Cu") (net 10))
 (segment (start 191.75 81.5) (end 189.8483 81.5) (width 0.2) (layer "F.Cu") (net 10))
 (segment (start 179.25 56.5) (end 181.1517 56.5) (width 0.2) (layer "F.Cu") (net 10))
 (segment (start 158.5 81.5) (end 160.4017 81.5) (width 0.2) (layer "F.Cu") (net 10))
 (segment (start 158.5 71.5) (end 160.4017 71.5) (width 0.2) (layer "F.Cu") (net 10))
 (segment (start 181.1517 71.5) (end 181.1517 81.5) (width 0.2) (layer "F.Cu") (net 10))
 (segment (start 189.8483 71.5) (end 189.8483 81.5) (width 0.2) (layer "B.Cu") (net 10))
 (segment (start 158.5 71.5) (end 171 71.5) (width 0.2) (layer "B.Cu") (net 10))
 (segment (start 189.8483 81.5) (end 179.25 81.5) (width 0.2) (layer "B.Cu") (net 10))
 (segment (start 191.75 71.5) (end 189.8483 71.5) (width 0.2) (layer "B.Cu") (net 10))
 (segment (start 179.25 71.5) (end 171 71.5) (width 0.2) (layer "B.Cu") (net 10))
 (segment (start 191.75 56.5) (end 179.25 56.5) (width 0.2) (layer "B.Cu") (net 10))
 (segment (start 172.9017 51.5) (end 172.9017 52.0534) (width 0.2) (layer "B.Cu") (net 10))
 (segment (start 172.9017 52.0534) (end 177.3483 56.5) (width 0.2) (layer "B.Cu") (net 10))
 (segment (start 191.75 81.5) (end 189.8483 81.5) (width 0.2) (layer "B.Cu") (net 10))
 (segment (start 158.5 51.5) (end 171 51.5) (width 0.2) (layer "B.Cu") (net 10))
 (segment (start 171 51.5) (end 172.9017 51.5) (width 0.2) (layer "B.Cu") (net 10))
 (segment (start 179.25 56.5) (end 177.3483 56.5) (width 0.2) (layer "B.Cu") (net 10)))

